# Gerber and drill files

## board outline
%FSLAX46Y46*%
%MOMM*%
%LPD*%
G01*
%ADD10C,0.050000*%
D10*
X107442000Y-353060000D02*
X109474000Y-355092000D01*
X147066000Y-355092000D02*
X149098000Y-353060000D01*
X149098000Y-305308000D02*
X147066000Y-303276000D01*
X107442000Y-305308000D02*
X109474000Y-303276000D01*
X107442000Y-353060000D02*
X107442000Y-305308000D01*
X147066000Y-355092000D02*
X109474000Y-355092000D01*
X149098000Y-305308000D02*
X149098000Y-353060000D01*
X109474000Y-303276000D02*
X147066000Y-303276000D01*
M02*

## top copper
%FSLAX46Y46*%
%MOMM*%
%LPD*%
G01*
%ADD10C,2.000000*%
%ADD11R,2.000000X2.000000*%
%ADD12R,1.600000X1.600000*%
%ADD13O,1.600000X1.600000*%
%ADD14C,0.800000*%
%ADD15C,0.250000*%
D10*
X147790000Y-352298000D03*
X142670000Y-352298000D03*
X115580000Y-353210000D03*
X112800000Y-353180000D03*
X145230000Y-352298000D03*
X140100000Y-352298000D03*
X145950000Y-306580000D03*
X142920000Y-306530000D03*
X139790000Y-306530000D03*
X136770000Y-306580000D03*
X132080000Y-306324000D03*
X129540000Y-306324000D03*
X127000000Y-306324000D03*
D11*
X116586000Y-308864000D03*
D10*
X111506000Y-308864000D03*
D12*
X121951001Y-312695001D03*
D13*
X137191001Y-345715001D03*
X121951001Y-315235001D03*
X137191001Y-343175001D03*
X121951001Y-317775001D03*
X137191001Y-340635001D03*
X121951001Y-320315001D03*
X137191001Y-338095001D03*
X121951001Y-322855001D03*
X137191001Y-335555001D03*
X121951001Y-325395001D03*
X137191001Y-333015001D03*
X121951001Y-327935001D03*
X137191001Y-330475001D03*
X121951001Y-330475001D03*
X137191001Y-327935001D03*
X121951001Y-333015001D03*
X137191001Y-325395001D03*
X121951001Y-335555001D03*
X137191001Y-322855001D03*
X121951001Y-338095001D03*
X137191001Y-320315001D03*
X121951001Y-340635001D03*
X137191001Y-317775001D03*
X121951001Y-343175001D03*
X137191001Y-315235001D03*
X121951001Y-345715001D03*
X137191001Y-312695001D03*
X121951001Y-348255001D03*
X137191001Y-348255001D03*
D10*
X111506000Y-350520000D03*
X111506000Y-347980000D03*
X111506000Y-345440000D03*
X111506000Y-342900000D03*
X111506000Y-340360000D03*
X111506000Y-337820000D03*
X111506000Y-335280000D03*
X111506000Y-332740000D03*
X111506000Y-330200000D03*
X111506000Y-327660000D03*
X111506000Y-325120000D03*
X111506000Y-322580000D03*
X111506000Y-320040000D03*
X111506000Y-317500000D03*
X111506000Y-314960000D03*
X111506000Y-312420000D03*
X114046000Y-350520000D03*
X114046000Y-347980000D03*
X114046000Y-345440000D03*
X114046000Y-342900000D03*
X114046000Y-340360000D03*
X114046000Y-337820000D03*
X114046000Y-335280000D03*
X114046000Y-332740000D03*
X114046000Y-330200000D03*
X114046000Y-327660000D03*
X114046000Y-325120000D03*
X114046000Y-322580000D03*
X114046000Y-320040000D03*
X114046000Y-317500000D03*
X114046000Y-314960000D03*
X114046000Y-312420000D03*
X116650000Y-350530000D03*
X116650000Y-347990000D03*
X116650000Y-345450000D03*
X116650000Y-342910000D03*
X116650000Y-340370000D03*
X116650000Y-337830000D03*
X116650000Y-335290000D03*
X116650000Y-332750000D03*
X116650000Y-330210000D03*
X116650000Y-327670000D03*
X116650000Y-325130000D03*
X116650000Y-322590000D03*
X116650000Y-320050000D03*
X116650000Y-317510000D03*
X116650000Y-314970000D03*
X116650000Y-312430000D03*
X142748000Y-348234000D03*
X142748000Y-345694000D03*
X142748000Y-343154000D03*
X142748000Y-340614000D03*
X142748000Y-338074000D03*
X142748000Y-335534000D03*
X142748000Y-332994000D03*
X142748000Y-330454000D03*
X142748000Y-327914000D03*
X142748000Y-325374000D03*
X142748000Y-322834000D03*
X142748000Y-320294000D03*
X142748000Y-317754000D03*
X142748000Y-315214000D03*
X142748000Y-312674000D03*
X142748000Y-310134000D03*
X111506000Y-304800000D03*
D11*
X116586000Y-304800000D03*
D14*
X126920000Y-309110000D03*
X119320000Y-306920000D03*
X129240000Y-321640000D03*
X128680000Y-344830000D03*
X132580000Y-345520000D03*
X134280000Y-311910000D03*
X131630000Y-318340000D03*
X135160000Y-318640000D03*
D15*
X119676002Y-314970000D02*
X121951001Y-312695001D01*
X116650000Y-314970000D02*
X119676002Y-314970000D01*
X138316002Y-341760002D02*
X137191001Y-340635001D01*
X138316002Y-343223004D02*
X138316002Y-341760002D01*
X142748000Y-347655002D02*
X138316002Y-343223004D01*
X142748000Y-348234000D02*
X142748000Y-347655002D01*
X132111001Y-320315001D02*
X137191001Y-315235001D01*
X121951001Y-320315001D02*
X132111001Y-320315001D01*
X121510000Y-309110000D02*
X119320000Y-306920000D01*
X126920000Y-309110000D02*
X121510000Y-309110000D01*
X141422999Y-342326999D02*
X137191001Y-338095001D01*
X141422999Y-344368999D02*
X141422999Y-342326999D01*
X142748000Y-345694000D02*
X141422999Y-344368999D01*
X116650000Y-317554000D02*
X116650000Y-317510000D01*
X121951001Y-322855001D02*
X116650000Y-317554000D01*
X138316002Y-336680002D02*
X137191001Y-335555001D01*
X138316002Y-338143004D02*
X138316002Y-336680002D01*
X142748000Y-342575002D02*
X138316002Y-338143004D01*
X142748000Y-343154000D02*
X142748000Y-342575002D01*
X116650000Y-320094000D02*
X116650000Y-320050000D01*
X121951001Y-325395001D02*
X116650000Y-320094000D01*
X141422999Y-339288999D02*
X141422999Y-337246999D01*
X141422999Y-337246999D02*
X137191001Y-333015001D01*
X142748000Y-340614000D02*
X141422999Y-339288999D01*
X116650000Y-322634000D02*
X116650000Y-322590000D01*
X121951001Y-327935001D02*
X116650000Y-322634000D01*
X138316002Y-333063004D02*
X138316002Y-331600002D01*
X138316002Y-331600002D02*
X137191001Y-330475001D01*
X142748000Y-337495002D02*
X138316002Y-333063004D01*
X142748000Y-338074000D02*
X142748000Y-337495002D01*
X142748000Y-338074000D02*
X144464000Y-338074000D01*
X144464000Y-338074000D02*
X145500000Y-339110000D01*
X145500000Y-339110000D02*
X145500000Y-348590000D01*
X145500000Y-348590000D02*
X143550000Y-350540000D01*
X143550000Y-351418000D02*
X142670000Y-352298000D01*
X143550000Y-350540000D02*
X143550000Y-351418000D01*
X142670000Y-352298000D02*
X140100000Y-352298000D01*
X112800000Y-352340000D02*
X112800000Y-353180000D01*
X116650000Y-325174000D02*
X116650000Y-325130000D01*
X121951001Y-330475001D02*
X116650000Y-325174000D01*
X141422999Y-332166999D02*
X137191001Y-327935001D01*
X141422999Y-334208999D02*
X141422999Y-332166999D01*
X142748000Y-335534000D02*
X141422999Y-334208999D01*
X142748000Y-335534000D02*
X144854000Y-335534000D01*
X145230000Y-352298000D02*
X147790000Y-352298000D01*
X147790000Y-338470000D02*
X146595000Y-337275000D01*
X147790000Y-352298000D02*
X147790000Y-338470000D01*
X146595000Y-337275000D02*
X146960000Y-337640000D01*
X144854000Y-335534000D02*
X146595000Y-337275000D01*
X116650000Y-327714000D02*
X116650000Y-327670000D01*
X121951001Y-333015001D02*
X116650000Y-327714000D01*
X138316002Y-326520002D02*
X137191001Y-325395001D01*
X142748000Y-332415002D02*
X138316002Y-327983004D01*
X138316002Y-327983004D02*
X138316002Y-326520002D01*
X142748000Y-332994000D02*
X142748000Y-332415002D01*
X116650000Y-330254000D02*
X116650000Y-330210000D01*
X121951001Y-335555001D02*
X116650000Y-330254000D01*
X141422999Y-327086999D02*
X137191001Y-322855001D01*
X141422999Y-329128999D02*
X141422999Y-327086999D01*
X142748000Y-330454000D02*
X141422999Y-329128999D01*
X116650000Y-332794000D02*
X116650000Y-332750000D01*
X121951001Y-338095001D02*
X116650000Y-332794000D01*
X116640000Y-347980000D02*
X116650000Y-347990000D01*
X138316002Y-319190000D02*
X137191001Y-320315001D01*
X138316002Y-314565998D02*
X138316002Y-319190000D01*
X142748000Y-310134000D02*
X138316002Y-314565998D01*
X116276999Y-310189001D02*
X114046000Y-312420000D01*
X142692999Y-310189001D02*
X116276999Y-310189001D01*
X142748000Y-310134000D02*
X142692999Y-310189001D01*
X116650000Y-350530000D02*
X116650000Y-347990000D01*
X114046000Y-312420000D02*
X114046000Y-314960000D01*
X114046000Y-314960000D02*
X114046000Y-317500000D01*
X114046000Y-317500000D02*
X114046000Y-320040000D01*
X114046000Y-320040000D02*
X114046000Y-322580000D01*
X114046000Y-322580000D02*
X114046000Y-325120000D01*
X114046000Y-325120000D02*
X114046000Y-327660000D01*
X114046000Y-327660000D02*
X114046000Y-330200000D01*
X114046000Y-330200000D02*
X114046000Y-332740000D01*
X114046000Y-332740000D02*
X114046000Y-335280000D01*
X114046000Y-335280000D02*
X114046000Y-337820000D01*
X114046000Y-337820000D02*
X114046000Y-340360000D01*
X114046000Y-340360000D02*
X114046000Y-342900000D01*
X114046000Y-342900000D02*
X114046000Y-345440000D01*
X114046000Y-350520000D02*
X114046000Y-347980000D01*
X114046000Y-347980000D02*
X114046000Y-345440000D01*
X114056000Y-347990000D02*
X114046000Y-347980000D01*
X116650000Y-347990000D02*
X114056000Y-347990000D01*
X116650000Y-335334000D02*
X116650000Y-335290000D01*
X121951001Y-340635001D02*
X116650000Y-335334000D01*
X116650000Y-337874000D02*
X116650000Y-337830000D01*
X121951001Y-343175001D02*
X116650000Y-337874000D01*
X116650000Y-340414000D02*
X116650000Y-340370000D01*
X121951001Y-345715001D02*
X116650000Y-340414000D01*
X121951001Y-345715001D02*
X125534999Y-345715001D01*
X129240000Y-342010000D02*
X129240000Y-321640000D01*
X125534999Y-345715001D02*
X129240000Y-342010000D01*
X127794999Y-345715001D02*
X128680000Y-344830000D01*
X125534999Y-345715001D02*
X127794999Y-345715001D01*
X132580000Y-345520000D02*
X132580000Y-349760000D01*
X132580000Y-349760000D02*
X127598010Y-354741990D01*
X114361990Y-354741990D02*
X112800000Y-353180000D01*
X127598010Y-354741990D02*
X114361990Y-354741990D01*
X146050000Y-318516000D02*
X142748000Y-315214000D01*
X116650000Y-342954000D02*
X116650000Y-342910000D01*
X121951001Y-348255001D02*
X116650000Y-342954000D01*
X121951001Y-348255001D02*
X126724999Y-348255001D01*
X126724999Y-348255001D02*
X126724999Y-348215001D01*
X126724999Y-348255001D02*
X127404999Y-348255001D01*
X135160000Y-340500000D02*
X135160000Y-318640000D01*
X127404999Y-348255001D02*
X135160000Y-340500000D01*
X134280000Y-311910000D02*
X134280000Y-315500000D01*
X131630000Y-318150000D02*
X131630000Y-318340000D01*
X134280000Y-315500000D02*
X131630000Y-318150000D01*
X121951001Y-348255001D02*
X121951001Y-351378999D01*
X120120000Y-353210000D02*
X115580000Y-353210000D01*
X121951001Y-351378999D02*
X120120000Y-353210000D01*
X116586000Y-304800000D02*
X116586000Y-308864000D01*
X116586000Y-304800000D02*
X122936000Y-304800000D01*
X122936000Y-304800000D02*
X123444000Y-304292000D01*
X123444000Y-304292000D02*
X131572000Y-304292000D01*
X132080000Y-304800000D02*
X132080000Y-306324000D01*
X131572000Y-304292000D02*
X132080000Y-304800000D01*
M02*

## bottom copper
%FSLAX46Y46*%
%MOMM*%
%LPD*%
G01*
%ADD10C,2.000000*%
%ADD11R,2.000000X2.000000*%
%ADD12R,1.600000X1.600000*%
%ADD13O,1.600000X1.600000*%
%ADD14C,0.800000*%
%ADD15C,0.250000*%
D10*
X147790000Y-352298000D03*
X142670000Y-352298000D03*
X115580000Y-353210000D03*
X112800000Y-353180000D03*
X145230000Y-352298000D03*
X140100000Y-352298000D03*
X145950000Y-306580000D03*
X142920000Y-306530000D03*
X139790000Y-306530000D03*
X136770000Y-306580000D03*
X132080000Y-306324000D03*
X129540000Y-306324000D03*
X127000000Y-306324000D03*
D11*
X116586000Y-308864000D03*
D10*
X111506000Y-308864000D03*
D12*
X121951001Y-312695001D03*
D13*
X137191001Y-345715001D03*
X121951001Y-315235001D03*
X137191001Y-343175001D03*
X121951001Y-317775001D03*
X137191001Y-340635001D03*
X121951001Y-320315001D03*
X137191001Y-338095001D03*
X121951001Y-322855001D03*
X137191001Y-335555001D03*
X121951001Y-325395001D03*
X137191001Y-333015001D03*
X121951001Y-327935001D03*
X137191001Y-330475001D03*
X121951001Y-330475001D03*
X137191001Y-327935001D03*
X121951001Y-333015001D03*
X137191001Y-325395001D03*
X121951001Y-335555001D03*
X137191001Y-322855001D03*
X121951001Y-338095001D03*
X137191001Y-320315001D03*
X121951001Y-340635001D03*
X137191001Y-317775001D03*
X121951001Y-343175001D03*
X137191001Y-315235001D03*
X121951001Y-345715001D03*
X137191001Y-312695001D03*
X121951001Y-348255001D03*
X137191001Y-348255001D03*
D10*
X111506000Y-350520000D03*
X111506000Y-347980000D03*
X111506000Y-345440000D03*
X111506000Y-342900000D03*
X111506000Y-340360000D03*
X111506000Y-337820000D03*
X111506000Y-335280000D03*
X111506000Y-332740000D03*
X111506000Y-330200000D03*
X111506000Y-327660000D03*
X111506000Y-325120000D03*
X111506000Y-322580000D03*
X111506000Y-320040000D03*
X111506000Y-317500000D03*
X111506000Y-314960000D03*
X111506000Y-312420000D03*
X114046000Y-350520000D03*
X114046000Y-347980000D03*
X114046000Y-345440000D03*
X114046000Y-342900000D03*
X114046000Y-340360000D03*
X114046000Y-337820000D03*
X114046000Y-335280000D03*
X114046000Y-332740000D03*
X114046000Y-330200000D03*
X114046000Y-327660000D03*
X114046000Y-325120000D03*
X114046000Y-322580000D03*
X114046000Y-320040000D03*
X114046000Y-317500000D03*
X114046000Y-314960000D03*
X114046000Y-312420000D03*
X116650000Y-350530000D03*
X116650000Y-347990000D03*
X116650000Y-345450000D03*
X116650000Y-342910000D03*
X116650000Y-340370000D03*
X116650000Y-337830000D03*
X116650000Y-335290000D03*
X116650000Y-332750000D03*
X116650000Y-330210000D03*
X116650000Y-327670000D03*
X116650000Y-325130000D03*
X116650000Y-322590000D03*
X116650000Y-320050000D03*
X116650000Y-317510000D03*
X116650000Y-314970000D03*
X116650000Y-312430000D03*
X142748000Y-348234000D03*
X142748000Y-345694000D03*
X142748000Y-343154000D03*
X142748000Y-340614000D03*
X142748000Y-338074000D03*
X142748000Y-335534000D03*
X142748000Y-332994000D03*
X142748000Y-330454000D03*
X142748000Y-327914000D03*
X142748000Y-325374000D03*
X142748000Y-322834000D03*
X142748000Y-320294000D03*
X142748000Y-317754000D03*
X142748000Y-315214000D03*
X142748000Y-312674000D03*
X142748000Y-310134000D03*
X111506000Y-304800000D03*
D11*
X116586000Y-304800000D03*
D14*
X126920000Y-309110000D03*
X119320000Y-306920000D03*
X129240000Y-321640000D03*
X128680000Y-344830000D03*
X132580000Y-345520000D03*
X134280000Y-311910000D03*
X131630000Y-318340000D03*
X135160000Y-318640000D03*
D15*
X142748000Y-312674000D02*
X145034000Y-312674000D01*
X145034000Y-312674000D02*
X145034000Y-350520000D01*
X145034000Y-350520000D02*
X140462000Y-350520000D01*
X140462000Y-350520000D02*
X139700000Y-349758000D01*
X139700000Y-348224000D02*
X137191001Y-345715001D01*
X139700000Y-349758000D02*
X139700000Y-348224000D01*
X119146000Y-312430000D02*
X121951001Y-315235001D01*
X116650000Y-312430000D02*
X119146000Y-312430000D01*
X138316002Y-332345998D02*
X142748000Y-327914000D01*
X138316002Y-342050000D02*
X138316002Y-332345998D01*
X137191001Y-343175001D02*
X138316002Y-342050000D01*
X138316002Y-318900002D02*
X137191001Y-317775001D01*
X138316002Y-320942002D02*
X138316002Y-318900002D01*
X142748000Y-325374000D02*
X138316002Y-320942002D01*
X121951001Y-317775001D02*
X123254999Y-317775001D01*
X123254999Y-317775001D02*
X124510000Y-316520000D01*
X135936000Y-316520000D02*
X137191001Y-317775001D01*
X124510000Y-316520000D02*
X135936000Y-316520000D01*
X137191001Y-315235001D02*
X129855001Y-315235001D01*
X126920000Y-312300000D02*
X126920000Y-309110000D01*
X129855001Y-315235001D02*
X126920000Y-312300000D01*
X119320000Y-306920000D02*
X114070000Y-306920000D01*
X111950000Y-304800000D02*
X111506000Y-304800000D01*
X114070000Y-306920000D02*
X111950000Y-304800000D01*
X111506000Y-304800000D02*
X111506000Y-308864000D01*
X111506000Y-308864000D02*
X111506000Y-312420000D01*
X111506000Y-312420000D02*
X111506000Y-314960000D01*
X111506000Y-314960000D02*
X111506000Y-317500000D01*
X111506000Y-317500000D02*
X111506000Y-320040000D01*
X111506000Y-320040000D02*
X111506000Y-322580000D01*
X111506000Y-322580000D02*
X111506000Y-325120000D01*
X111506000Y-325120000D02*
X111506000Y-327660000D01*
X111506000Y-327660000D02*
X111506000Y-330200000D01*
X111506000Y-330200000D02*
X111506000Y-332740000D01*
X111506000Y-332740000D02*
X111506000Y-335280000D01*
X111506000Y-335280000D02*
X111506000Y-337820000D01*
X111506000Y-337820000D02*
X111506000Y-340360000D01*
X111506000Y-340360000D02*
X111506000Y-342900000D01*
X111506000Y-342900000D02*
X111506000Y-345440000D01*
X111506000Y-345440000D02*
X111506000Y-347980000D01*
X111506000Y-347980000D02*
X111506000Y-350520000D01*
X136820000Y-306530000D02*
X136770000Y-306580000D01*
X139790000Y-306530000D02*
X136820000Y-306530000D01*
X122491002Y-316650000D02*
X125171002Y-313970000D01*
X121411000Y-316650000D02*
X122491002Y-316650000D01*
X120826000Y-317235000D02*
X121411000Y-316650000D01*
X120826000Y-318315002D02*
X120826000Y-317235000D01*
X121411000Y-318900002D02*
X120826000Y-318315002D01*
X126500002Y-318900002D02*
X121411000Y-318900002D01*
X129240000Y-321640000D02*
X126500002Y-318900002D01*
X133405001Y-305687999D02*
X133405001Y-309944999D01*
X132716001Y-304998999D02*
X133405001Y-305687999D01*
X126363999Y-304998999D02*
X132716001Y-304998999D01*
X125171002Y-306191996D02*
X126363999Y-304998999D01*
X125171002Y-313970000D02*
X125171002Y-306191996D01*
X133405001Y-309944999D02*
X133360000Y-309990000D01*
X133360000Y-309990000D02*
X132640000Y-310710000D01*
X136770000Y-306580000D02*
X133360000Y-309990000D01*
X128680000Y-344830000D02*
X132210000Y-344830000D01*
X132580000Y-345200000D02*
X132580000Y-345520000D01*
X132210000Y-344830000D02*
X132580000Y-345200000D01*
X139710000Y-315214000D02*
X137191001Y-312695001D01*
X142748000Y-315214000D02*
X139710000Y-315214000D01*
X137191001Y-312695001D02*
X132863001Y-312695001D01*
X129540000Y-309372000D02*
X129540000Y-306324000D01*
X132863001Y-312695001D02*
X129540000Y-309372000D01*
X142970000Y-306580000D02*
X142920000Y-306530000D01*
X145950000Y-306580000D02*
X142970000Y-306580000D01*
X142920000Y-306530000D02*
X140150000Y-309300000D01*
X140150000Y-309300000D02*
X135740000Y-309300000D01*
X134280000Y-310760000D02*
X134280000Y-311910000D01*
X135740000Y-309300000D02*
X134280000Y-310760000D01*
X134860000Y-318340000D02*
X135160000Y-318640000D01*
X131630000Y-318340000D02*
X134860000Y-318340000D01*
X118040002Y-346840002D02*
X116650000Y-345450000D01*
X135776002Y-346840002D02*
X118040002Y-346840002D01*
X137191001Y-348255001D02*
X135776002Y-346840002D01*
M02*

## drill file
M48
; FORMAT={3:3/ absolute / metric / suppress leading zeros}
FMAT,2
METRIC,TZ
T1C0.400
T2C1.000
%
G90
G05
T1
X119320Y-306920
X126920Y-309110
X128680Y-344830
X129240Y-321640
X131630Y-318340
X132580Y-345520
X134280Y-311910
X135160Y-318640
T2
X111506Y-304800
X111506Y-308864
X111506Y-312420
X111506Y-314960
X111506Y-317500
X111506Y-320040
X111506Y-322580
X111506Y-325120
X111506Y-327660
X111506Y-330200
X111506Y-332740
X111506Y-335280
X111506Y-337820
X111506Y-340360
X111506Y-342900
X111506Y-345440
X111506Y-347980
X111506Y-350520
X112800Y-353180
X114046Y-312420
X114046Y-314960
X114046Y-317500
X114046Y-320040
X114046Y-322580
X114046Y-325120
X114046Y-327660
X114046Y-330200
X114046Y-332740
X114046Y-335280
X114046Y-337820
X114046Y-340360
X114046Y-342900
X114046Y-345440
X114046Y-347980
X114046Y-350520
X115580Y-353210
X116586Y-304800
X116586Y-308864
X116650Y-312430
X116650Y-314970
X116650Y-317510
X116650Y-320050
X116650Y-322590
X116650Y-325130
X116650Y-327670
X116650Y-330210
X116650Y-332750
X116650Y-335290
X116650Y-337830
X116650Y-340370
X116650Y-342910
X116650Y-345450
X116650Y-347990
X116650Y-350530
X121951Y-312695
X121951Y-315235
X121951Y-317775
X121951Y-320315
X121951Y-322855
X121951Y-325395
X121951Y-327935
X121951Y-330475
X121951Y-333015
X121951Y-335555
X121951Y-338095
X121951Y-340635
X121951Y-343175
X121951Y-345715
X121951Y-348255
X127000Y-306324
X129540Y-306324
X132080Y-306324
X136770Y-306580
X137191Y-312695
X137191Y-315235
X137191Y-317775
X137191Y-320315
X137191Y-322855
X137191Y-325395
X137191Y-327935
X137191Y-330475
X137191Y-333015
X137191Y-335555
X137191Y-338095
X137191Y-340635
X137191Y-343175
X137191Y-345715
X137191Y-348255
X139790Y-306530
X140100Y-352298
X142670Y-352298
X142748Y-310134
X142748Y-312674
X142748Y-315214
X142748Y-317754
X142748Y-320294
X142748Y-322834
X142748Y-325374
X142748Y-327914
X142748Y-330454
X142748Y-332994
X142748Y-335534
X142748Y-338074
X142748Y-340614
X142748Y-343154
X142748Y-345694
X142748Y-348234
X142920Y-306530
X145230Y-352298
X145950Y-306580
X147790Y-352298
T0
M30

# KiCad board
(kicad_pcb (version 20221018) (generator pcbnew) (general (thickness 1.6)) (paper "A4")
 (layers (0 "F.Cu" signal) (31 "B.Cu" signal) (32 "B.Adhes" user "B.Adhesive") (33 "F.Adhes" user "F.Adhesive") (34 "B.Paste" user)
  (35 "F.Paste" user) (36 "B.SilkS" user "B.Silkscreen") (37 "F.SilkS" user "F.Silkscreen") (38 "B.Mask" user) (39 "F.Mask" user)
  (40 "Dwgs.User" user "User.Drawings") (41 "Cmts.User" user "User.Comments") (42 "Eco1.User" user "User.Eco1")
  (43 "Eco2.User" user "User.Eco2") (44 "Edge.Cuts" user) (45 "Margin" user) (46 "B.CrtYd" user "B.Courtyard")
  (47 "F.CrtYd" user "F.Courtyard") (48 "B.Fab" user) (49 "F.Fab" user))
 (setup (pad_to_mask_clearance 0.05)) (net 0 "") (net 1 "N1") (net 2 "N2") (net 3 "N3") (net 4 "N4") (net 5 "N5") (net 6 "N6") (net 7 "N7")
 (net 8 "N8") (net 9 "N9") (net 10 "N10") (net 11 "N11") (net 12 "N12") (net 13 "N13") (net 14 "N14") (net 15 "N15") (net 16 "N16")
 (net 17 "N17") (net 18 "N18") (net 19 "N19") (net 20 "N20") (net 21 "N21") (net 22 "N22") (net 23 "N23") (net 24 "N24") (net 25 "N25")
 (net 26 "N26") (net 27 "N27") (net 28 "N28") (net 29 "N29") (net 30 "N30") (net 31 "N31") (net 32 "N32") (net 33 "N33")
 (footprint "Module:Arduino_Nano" (layer "F.Cu") (at 121.951001 312.695001)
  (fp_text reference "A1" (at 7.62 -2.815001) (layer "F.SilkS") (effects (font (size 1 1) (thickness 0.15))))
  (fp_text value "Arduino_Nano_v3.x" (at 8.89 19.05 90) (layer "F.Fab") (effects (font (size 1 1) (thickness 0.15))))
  (pad "1" thru_hole rect (at 0 0) (size 1.6 1.6) (drill 1) (layers "*.Cu" "*.Mask") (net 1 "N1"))
  (pad "2" thru_hole oval (at 0 2.54) (size 1.6 1.6) (drill 1) (layers "*.Cu" "*.Mask") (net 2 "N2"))
  (pad "3" thru_hole oval (at 0 5.08) (size 1.6 1.6) (drill 1) (layers "*.Cu" "*.Mask") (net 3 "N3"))
  (pad "4" thru_hole oval (at 0 7.62) (size 1.6 1.6) (drill 1) (layers "*.Cu" "*.Mask") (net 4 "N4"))
  (pad "5" thru_hole oval (at 0 10.16) (size 1.6 1.6) (drill 1) (layers "*.Cu" "*.Mask") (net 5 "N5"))
  (pad "6" thru_hole oval (at 0 12.7) (size 1.6 1.6) (drill 1) (layers "*.Cu" "*.Mask") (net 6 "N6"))
  (pad "7" thru_hole oval (at 0 15.24) (size 1.6 1.6) (drill 1) (layers "*.Cu" "*.Mask") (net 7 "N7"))
  (pad "8" thru_hole oval (at 0 17.78) (size 1.6 1.6) (drill 1) (layers "*.Cu" "*.Mask") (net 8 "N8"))
  (pad "9" thru_hole oval (at 0 20.32) (size 1.6 1.6) (drill 1) (layers "*.Cu" "*.Mask") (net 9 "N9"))
  (pad "10" thru_hole oval (at 0 22.86) (size 1.6 1.6) (drill 1) (layers "*.Cu" "*.Mask") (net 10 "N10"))
  (pad "11" thru_hole oval (at 0 25.4) (size 1.6 1.6) (drill 1) (layers "*.Cu" "*.Mask") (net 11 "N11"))
  (pad "12" thru_hole oval (at 0 27.94) (size 1.6 1.6) (drill 1) (layers "*.Cu" "*.Mask") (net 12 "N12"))
  (pad "13" thru_hole oval (at 0 30.48) (size 1.6 1.6) (drill 1) (layers "*.Cu" "*.Mask") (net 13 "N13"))
  (pad "14" thru_hole oval (at 0 33.02) (size 1.6 1.6) (drill 1) (layers "*.Cu" "*.Mask") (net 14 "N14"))
  (pad "15" thru_hole oval (at 0 35.56) (size 1.6 1.6) (drill 1) (layers "*.Cu" "*.Mask") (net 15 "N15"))
  (pad "16" thru_hole oval (at 15.24 35.56) (size 1.6 1.6) (drill 1) (layers "*.Cu" "*.Mask") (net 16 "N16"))
  (pad "17" thru_hole oval (at 15.24 33.02) (size 1.6 1.6) (drill 1) (layers "*.Cu" "*.Mask") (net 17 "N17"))
  (pad "18" thru_hole oval (at 15.24 30.48) (size 1.6 1.6) (drill 1) (layers "*.Cu" "*.Mask") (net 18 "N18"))
  (pad "19" thru_hole oval (at 15.24 27.94) (size 1.6 1.6) (drill 1) (layers "*.Cu" "*.Mask") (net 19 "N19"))
  (pad "20" thru_hole oval (at 15.24 25.4) (size 1.6 1.6) (drill 1) (layers "*.Cu" "*.Mask") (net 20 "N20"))
  (pad "21" thru_hole oval (at 15.24 22.86) (size 1.6 1.6) (drill 1) (layers "*.Cu" "*.Mask") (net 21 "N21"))
  (pad "22" thru_hole oval (at 15.24 20.32) (size 1.6 1.6) (drill 1) (layers "*.Cu" "*.Mask") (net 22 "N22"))
  (pad "23" thru_hole oval (at 15.24 17.78) (size 1.6 1.6) (drill 1) (layers "*.Cu" "*.Mask") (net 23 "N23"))
  (pad "24" thru_hole oval (at 15.24 15.24) (size 1.6 1.6) (drill 1) (layers "*.Cu" "*.Mask") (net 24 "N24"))
  (pad "25" thru_hole oval (at 15.24 12.7) (size 1.6 1.6) (drill 1) (layers "*.Cu" "*.Mask") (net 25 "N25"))
  (pad "26" thru_hole oval (at 15.24 10.16) (size 1.6 1.6) (drill 1) (layers "*.Cu" "*.Mask") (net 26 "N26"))
  (pad "27" thru_hole oval (at 15.24 7.62) (size 1.6 1.6) (drill 1) (layers "*.Cu" "*.Mask") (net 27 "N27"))
  (pad "28" thru_hole oval (at 15.24 5.08) (size 1.6 1.6) (drill 1) (layers "*.Cu" "*.Mask") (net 3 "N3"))
  (pad "29" thru_hole oval (at 15.24 2.54) (size 1.6 1.6) (drill 1) (layers "*.Cu" "*.Mask") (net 4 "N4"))
  (pad "30" thru_hole oval (at 15.24 0) (size 1.6 1.6) (drill 1) (layers "*.Cu" "*.Mask") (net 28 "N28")))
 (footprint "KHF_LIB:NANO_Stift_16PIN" (layer "F.Cu") (at 114.046 312.42 -90)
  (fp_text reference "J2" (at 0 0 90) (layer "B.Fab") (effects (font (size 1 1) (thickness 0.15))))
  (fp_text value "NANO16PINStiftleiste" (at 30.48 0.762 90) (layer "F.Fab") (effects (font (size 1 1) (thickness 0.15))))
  (pad "1" thru_hole circle (at 0 0 270) (size 2 2) (drill 1) (layers "*.Cu" "*.Mask") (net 27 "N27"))
  (pad "2" thru_hole circle (at 2.54 0 270) (size 2 2) (drill 1) (layers "*.Cu" "*.Mask") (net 27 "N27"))
  (pad "3" thru_hole circle (at 5.08 0 270) (size 2 2) (drill 1) (layers "*.Cu" "*.Mask") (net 27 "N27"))
  (pad "4" thru_hole circle (at 7.62 0 270) (size 2 2) (drill 1) (layers "*.Cu" "*.Mask") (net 27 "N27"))
  (pad "5" thru_hole circle (at 10.16 0 270) (size 2 2) (drill 1) (layers "*.Cu" "*.Mask") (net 27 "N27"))
  (pad "6" thru_hole circle (at 12.7 0 270) (size 2 2) (drill 1) (layers "*.Cu" "*.Mask") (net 27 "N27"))
  (pad "7" thru_hole circle (at 15.24 0 270) (size 2 2) (drill 1) (layers "*.Cu" "*.Mask") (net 27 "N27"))
  (pad "8" thru_hole circle (at 17.78 0 270) (size 2 2) (drill 1) (layers "*.Cu" "*.Mask") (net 27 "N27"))
  (pad "9" thru_hole circle (at 20.32 0 270) (size 2 2) (drill 1) (layers "*.Cu" "*.Mask") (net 27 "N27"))
  (pad "10" thru_hole circle (at 22.86 0 270) (size 2 2) (drill 1) (layers "*.Cu" "*.Mask") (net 27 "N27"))
  (pad "11" thru_hole circle (at 25.4 0 270) (size 2 2) (drill 1) (layers "*.Cu" "*.Mask") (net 27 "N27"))
  (pad "12" thru_hole circle (at 27.94 0 270) (size 2 2) (drill 1) (layers "*.Cu" "*.Mask") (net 27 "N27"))
  (pad "13" thru_hole circle (at 30.48 0 270) (size 2 2) (drill 1) (layers "*.Cu" "*.Mask") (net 27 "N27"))
  (pad "14" thru_hole circle (at 33.02 0 270) (size 2 2) (drill 1) (layers "*.Cu" "*.Mask") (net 27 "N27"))
  (pad "15" thru_hole circle (at 35.56 0 270) (size 2 2) (drill 1) (layers "*.Cu" "*.Mask") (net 27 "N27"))
  (pad "16" thru_hole circle (at 38.1 0 270) (size 2 2) (drill 1) (layers "*.Cu" "*.Mask") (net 27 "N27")))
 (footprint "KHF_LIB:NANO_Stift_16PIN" (layer "F.Cu") (at 116.65 312.43 -90)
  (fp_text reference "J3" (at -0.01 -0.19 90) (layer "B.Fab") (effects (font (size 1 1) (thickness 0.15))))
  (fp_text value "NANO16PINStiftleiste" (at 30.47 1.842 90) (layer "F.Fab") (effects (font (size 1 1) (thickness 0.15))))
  (pad "1" thru_hole circle (at 0 0 270) (size 2 2) (drill 1) (layers "*.Cu" "*.Mask") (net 2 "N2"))
  (pad "2" thru_hole circle (at 2.54 0 270) (size 2 2) (drill 1) (layers "*.Cu" "*.Mask") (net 1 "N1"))
  (pad "3" thru_hole circle (at 5.08 0 270) (size 2 2) (drill 1) (layers "*.Cu" "*.Mask") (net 5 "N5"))
  (pad "4" thru_hole circle (at 7.62 0 270) (size 2 2) (drill 1) (layers "*.Cu" "*.Mask") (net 6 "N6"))
  (pad "5" thru_hole circle (at 10.16 0 270) (size 2 2) (drill 1) (layers "*.Cu" "*.Mask") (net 7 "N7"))
  (pad "6" thru_hole circle (at 12.7 0 270) (size 2 2) (drill 1) (layers "*.Cu" "*.Mask") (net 8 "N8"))
  (pad "7" thru_hole circle (at 15.24 0 270) (size 2 2) (drill 1) (layers "*.Cu" "*.Mask") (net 9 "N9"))
  (pad "8" thru_hole circle (at 17.78 0 270) (size 2 2) (drill 1) (layers "*.Cu" "*.Mask") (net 10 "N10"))
  (pad "9" thru_hole circle (at 20.32 0 270) (size 2 2) (drill 1) (layers "*.Cu" "*.Mask") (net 11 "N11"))
  (pad "10" thru_hole circle (at 22.86 0 270) (size 2 2) (drill 1) (layers "*.Cu" "*.Mask") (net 12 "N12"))
  (pad "11" thru_hole circle (at 25.4 0 270) (size 2 2) (drill 1) (layers "*.Cu" "*.Mask") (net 13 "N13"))
  (pad "12" thru_hole circle (at 27.94 0 270) (size 2 2) (drill 1) (layers "*.Cu" "*.Mask") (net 14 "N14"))
  (pad "13" thru_hole circle (at 30.48 0 270) (size 2 2) (drill 1) (layers "*.Cu" "*.Mask") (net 15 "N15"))
  (pad "14" thru_hole circle (at 33.02 0 270) (size 2 2) (drill 1) (layers "*.Cu" "*.Mask") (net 16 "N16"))
  (pad "15" thru_hole circle (at 35.56 0 270) (size 2 2) (drill 1) (layers "*.Cu" "*.Mask") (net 27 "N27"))
  (pad "16" thru_hole circle (at 38.1 0 270) (size 2 2) (drill 1) (layers "*.Cu" "*.Mask") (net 27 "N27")))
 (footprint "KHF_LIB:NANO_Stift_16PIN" (layer "F.Cu") (at 142.748 348.234 90)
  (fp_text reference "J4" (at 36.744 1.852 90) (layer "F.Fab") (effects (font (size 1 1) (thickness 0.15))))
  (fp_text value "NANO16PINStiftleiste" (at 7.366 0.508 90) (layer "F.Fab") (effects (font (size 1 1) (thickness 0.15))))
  (pad "1" thru_hole circle (at 0 0 90) (size 2 2) (drill 1) (layers "*.Cu" "*.Mask") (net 19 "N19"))
  (pad "2" thru_hole circle (at 2.54 0 90) (size 2 2) (drill 1) (layers "*.Cu" "*.Mask") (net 20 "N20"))
  (pad "3" thru_hole circle (at 5.08 0 90) (size 2 2) (drill 1) (layers "*.Cu" "*.Mask") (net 21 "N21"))
  (pad "4" thru_hole circle (at 7.62 0 90) (size 2 2) (drill 1) (layers "*.Cu" "*.Mask") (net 22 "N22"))
  (pad "5" thru_hole circle (at 10.16 0 90) (size 2 2) (drill 1) (layers "*.Cu" "*.Mask") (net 23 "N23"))
  (pad "6" thru_hole circle (at 12.7 0 90) (size 2 2) (drill 1) (layers "*.Cu" "*.Mask") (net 24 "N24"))
  (pad "7" thru_hole circle (at 15.24 0 90) (size 2 2) (drill 1) (layers "*.Cu" "*.Mask") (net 25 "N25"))
  (pad "8" thru_hole circle (at 17.78 0 90) (size 2 2) (drill 1) (layers "*.Cu" "*.Mask") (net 26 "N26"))
  (pad "9" thru_hole circle (at 20.32 0 90) (size 2 2) (drill 1) (layers "*.Cu" "*.Mask") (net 18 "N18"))
  (pad "10" thru_hole circle (at 22.86 0 90) (size 2 2) (drill 1) (layers "*.Cu" "*.Mask") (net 3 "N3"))
  (pad "11" thru_hole circle (at 25.4 0 90) (size 2 2) (drill 1) (layers "*.Cu" "*.Mask") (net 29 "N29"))
  (pad "12" thru_hole circle (at 27.94 0 90) (size 2 2) (drill 1) (layers "*.Cu" "*.Mask") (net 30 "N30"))
  (pad "13" thru_hole circle (at 30.48 0 90) (size 2 2) (drill 1) (layers "*.Cu" "*.Mask") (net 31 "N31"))
  (pad "14" thru_hole circle (at 33.02 0 90) (size 2 2) (drill 1) (layers "*.Cu" "*.Mask") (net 28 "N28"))
  (pad "15" thru_hole circle (at 35.56 0 90) (size 2 2) (drill 1) (layers "*.Cu" "*.Mask") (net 17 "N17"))
  (pad "16" thru_hole circle (at 38.1 0 90) (size 2 2) (drill 1) (layers "*.Cu" "*.Mask") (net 27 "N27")))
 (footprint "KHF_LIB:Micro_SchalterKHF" (layer "F.Cu") (at 132.08 306.324 180)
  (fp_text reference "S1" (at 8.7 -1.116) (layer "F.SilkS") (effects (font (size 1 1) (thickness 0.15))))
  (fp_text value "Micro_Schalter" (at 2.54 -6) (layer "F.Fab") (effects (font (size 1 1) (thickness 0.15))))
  (pad "1" thru_hole circle (at 0 0 180) (size 2 2) (drill 1) (layers "*.Cu" "*.Mask") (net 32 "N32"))
  (pad "2" thru_hole circle (at 2.54 0 180) (size 2 2) (drill 1) (layers "*.Cu" "*.Mask") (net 28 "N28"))
  (pad "3" thru_hole circle (at 5.08 0 180) (size 2 2) (drill 1) (layers "*.Cu" "*.Mask") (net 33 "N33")))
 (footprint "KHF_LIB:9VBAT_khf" (layer "F.Cu") (at 111.506 304.8)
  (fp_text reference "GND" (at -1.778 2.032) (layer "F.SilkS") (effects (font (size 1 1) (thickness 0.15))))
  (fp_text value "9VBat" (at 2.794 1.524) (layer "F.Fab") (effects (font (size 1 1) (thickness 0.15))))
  (pad "1" thru_hole circle (at 0 0) (size 2 2) (drill 1) (layers "*.Cu" "*.Mask") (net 4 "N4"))
  (pad "2" thru_hole rect (at 5.08 0) (size 2 2) (drill 1) (layers "*.Cu" "*.Mask") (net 32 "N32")))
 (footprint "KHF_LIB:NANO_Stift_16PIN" (layer "F.Cu") (at 111.506 350.52 90)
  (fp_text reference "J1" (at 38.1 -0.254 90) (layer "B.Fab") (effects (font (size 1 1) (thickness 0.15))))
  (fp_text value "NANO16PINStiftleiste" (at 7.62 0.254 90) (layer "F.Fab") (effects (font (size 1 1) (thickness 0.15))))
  (pad "1" thru_hole circle (at 0 0 90) (size 2 2) (drill 1) (layers "*.Cu" "*.Mask") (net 4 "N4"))
  (pad "2" thru_hole circle (at 2.54 0 90) (size 2 2) (drill 1) (layers "*.Cu" "*.Mask") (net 4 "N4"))
  (pad "3" thru_hole circle (at 5.08 0 90) (size 2 2) (drill 1) (layers "*.Cu" "*.Mask") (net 4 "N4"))
  (pad "4" thru_hole circle (at 7.62 0 90) (size 2 2) (drill 1) (layers "*.Cu" "*.Mask") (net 4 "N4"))
  (pad "5" thru_hole circle (at 10.16 0 90) (size 2 2) (drill 1) (layers "*.Cu" "*.Mask") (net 4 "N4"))
  (pad "6" thru_hole circle (at 12.7 0 90) (size 2 2) (drill 1) (layers "*.Cu" "*.Mask") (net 4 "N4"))
  (pad "7" thru_hole circle (at 15.24 0 90) (size 2 2) (drill 1) (layers "*.Cu" "*.Mask") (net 4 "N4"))
  (pad "8" thru_hole circle (at 17.78 0 90) (size 2 2) (drill 1) (layers "*.Cu" "*.Mask") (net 4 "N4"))
  (pad "9" thru_hole circle (at 20.32 0 90) (size 2 2) (drill 1) (layers "*.Cu" "*.Mask") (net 4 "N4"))
  (pad "10" thru_hole circle (at 22.86 0 90) (size 2 2) (drill 1) (layers "*.Cu" "*.Mask") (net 4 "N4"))
  (pad "11" thru_hole circle (at 25.4 0 90) (size 2 2) (drill 1) (layers "*.Cu" "*.Mask") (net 4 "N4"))
  (pad "12" thru_hole circle (at 27.94 0 90) (size 2 2) (drill 1) (layers "*.Cu" "*.Mask") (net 4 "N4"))
  (pad "13" thru_hole circle (at 30.48 0 90) (size 2 2) (drill 1) (layers "*.Cu" "*.Mask") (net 4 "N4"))
  (pad "14" thru_hole circle (at 33.02 0 90) (size 2 2) (drill 1) (layers "*.Cu" "*.Mask") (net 4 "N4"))
  (pad "15" thru_hole circle (at 35.56 0 90) (size 2 2) (drill 1) (layers "*.Cu" "*.Mask") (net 4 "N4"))
  (pad "16" thru_hole circle (at 38.1 0 90) (size 2 2) (drill 1) (layers "*.Cu" "*.Mask") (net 4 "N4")))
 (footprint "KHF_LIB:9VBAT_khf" (layer "F.Cu") (at 111.506 308.864)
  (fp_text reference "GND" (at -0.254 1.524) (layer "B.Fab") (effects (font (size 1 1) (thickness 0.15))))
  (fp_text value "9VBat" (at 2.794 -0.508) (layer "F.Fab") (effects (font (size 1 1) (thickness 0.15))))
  (pad "1" thru_hole circle (at 0 0) (size 2 2) (drill 1) (layers "*.Cu" "*.Mask") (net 4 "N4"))
  (pad "2" thru_hole rect (at 5.08 0) (size 2 2) (drill 1) (layers "*.Cu" "*.Mask") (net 32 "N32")))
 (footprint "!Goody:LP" (layer "F.Cu") (at 137.31 305.93)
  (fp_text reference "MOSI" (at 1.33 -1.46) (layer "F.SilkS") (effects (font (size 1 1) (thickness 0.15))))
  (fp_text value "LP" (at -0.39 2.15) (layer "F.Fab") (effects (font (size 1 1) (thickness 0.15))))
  (pad "1" thru_hole circle (at -0.54 0.65) (size 2 2) (drill 1) (layers "*.Cu" "*.Mask") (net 14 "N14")))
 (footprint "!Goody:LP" (layer "F.Cu") (at 145.77 351.648)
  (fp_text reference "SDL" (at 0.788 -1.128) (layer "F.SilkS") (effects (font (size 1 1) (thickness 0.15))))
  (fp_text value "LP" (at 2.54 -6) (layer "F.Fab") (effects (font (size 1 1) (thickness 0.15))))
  (pad "1" thru_hole circle (at -0.54 0.65) (size 2 2) (drill 1) (layers "*.Cu" "*.Mask") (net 24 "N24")))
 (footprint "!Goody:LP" (layer "F.Cu") (at 116.12 352.56)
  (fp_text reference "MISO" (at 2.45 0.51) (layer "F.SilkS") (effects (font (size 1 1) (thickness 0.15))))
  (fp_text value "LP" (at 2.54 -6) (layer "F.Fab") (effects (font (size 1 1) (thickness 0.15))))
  (pad "1" thru_hole circle (at -0.54 0.65) (size 2 2) (drill 1) (layers "*.Cu" "*.Mask") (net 15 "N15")))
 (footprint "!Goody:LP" (layer "F.Cu") (at 148.33 351.648)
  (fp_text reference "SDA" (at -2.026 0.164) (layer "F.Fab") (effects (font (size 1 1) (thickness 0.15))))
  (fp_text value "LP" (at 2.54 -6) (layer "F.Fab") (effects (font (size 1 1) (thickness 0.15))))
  (pad "1" thru_hole circle (at -0.54 0.65) (size 2 2) (drill 1) (layers "*.Cu" "*.Mask") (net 24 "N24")))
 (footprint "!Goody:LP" (layer "F.Cu") (at 140.64 351.648)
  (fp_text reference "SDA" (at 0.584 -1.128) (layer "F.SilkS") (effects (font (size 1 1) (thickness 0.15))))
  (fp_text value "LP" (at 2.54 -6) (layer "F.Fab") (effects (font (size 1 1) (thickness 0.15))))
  (pad "1" thru_hole circle (at -0.54 0.65) (size 2 2) (drill 1) (layers "*.Cu" "*.Mask") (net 23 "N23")))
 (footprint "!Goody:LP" (layer "F.Cu") (at 143.21 351.648)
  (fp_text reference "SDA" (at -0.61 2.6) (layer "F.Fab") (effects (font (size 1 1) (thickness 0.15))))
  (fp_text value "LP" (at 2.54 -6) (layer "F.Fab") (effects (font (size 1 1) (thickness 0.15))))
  (pad "1" thru_hole circle (at -0.54 0.65) (size 2 2) (drill 1) (layers "*.Cu" "*.Mask") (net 23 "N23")))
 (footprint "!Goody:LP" (layer "F.Cu") (at 113.34 352.53)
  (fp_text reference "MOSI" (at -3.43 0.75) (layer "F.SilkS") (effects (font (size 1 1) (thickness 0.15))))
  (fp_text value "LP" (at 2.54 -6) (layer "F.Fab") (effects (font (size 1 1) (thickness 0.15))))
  (pad "1" thru_hole circle (at -0.54 0.65) (size 2 2) (drill 1) (layers "*.Cu" "*.Mask") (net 14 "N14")))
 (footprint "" (layer "F.Cu") (at 112.268 348.488)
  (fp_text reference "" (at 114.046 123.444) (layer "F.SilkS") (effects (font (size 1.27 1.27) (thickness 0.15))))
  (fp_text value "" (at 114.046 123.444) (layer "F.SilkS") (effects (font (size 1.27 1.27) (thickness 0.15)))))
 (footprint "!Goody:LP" (layer "F.Cu") (at 146.49 305.93)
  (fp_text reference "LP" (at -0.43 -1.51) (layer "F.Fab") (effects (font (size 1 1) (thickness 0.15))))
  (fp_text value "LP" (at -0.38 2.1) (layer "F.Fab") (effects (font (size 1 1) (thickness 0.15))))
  (pad "1" thru_hole circle (at -0.54 0.65) (size 2 2) (drill 1) (layers "*.Cu" "*.Mask") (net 15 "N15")))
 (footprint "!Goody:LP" (layer "F.Cu") (at 143.46 305.88)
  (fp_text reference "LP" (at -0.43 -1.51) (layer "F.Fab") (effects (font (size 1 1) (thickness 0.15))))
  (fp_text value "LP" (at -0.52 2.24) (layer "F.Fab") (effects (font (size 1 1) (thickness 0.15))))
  (pad "1" thru_hole circle (at -0.54 0.65) (size 2 2) (drill 1) (layers "*.Cu" "*.Mask") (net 15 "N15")))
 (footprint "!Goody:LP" (layer "F.Cu") (at 140.33 305.88)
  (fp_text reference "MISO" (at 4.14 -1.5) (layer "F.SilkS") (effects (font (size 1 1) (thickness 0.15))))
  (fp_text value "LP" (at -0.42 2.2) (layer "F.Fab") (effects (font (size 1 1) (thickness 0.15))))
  (pad "1" thru_hole circle (at -0.54 0.65) (size 2 2) (drill 1) (layers "*.Cu" "*.Mask") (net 14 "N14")))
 (gr_line (start 107.442 353.06) (end 107.442 305.308) (stroke (width 0.05) (type solid)) (layer "Edge.Cuts"))
 (gr_line (start 147.066 355.092) (end 149.098 353.06) (stroke (width 0.05) (type solid)) (layer "Edge.Cuts"))
 (gr_line (start 147.066 355.092) (end 109.474 355.092) (stroke (width 0.05) (type solid)) (layer "Edge.Cuts"))
 (gr_line (start 107.442 305.308) (end 109.474 303.276) (stroke (width 0.05) (type solid)) (layer "Edge.Cuts"))
 (gr_line (start 107.442 353.06) (end 109.474 355.092) (stroke (width 0.05) (type solid)) (layer "Edge.Cuts"))
 (gr_line (start 149.098 305.308) (end 147.066 303.276) (stroke (width 0.05) (type solid)) (layer "Edge.Cuts"))
 (gr_line (start 149.098 305.308) (end 149.098 353.06) (stroke (width 0.05) (type solid)) (layer "Edge.Cuts"))
 (gr_line (start 109.474 303.276) (end 147.066 303.276) (stroke (width 0.05) (type solid)) (layer "Edge.Cuts"))
 (segment (start 119.676002 314.97) (end 121.951001 312.695001) (width 0.25) (layer "F.Cu") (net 1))
 (segment (start 116.65 314.97) (end 119.676002 314.97) (width 0.25) (layer "F.Cu") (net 1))
 (segment (start 140.462 350.52) (end 139.7 349.758) (width 0.25) (layer "B.Cu") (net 17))
 (segment (start 145.034 312.674) (end 145.034 350.52) (width 0.25) (layer "B.Cu") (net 17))
 (segment (start 139.7 348.224) (end 137.191001 345.715001) (width 0.25) (layer "B.Cu") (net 17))
 (segment (start 145.034 350.52) (end 140.462 350.52) (width 0.25) (layer "B.Cu") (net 17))
 (segment (start 142.748 312.674) (end 145.034 312.674) (width 0.25) (layer "B.Cu") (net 17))
 (segment (start 139.7 349.758) (end 139.7 348.224) (width 0.25) (layer "B.Cu") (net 17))
 (segment (start 119.146 312.43) (end 121.951001 315.235001) (width 0.25) (layer "B.Cu") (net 2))
 (segment (start 116.65 312.43) (end 119.146 312.43) (width 0.25) (layer "B.Cu") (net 2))
 (segment (start 137.191001 343.175001) (end 138.316002 342.05) (width 0.25) (layer "B.Cu") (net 18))
 (segment (start 138.316002 332.345998) (end 142.748 327.914) (width 0.25) (layer "B.Cu") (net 18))
 (segment (start 138.316002 342.05) (end 138.316002 332.345998) (width 0.25) (layer "B.Cu") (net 18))
 (segment (start 138.316002 318.900002) (end 137.191001 317.775001) (width 0.25) (layer "B.Cu") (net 3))
 (segment (start 138.316002 320.942002) (end 138.316002 318.900002) (width 0.25) (layer "B.Cu") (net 3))
 (segment (start 123.254999 317.775001) (end 124.51 316.52) (width 0.25) (layer "B.Cu") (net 3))
 (segment (start 121.951001 317.775001) (end 123.254999 317.775001) (width 0.25) (layer "B.Cu") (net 3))
 (segment (start 142.748 325.374) (end 138.316002 320.942002) (width 0.25) (layer "B.Cu") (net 3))
 (segment (start 135.936 316.52) (end 137.191001 317.775001) (width 0.25) (layer "B.Cu") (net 3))
 (segment (start 124.51 316.52) (end 135.936 316.52) (width 0.25) (layer "B.Cu") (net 3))
 (segment (start 142.748 347.655002) (end 138.316002 343.223004) (width 0.25) (layer "F.Cu") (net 19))
 (segment (start 138.316002 343.223004) (end 138.316002 341.760002) (width 0.25) (layer "F.Cu") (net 19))
 (segment (start 142.748 348.234) (end 142.748 347.655002) (width 0.25) (layer "F.Cu") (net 19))
 (segment (start 138.316002 341.760002) (end 137.191001 340.635001) (width 0.25) (layer "F.Cu") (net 19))
 (segment (start 121.951001 320.315001) (end 132.111001 320.315001) (width 0.25) (layer "F.Cu") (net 4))
 (segment (start 132.111001 320.315001) (end 137.191001 315.235001) (width 0.25) (layer "F.Cu") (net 4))
 (segment (start 121.51 309.11) (end 119.32 306.92) (width 0.25) (layer "F.Cu") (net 4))
 (segment (start 126.92 309.11) (end 121.51 309.11) (width 0.25) (layer "F.Cu") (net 4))
 (via (at 126.92 309.11) (size 0.8) (drill 0.4) (layers "F.Cu" "B.Cu") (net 4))
 (via (at 119.32 306.92) (size 0.8) (drill 0.4) (layers "F.Cu" "B.Cu") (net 4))
 (segment (start 111.506 337.82) (end 111.506 340.36) (width 0.25) (layer "B.Cu") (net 4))
 (segment (start 111.95 304.8) (end 111.506 304.8) (width 0.25) (layer "B.Cu") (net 4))
 (segment (start 111.506 308.864) (end 111.506 312.42) (width 0.25) (layer "B.Cu") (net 4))
 (segment (start 114.07 306.92) (end 111.95 304.8) (width 0.25) (layer "B.Cu") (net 4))
 (segment (start 111.506 320.04) (end 111.506 322.58) (width 0.25) (layer "B.Cu") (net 4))
 (segment (start 111.506 332.74) (end 111.506 335.28) (width 0.25) (layer "B.Cu") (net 4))
 (segment (start 111.506 304.8) (end 111.506 308.864) (width 0.25) (layer "B.Cu") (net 4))
 (segment (start 111.506 325.12) (end 111.506 327.66) (width 0.25) (layer "B.Cu") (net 4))
 (segment (start 111.506 342.9) (end 111.506 345.44) (width 0.25) (layer "B.Cu") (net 4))
 (segment (start 111.506 322.58) (end 111.506 325.12) (width 0.25) (layer "B.Cu") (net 4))
 (segment (start 119.32 306.92) (end 114.07 306.92) (width 0.25) (layer "B.Cu") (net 4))
 (segment (start 129.855001 315.235001) (end 126.92 312.3) (width 0.25) (layer "B.Cu") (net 4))
 (segment (start 111.506 314.96) (end 111.506 317.5) (width 0.25) (layer "B.Cu") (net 4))
 (segment (start 111.506 330.2) (end 111.506 332.74) (width 0.25) (layer "B.Cu") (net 4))
 (segment (start 137.191001 315.235001) (end 129.855001 315.235001) (width 0.25) (layer "B.Cu") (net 4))
 (segment (start 111.506 347.98) (end 111.506 350.52) (width 0.25) (layer "B.Cu") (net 4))
 (segment (start 111.506 317.5) (end 111.506 320.04) (width 0.25) (layer "B.Cu") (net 4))
 (segment (start 111.506 345.44) (end 111.506 347.98) (width 0.25) (layer "B.Cu") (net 4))
 (segment (start 111.506 312.42) (end 111.506 314.96) (width 0.25) (layer "B.Cu") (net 4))
 (segment (start 111.506 340.36) (end 111.506 342.9) (width 0.25) (layer "B.Cu") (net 4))
 (segment (start 111.506 335.28) (end 111.506 337.82) (width 0.25) (layer "B.Cu") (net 4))
 (segment (start 111.506 327.66) (end 111.506 330.2) (width 0.25) (layer "B.Cu") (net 4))
 (segment (start 126.92 312.3) (end 126.92 309.11) (width 0.25) (layer "B.Cu") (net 4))
 (segment (start 141.422999 342.326999) (end 137.191001 338.095001) (width 0.25) (layer "F.Cu") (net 20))
 (segment (start 141.422999 344.368999) (end 141.422999 342.326999) (width 0.25) (layer "F.Cu") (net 20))
 (segment (start 142.748 345.694) (end 141.422999 344.368999) (width 0.25) (layer "F.Cu") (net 20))
 (segment (start 121.951001 322.855001) (end 116.65 317.554) (width 0.25) (layer "F.Cu") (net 5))
 (segment (start 116.65 317.554) (end 116.65 317.51) (width 0.25) (layer "F.Cu") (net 5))
 (segment (start 138.316002 336.680002) (end 137.191001 335.555001) (width 0.25) (layer "F.Cu") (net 21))
 (segment (start 138.316002 338.143004) (end 138.316002 336.680002) (width 0.25) (layer "F.Cu") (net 21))
 (segment (start 142.748 343.154) (end 142.748 342.575002) (width 0.25) (layer "F.Cu") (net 21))
 (segment (start 142.748 342.575002) (end 138.316002 338.143004) (width 0.25) (layer "F.Cu") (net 21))
 (segment (start 116.65 320.094) (end 116.65 320.05) (width 0.25) (layer "F.Cu") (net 6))
 (segment (start 121.951001 325.395001) (end 116.65 320.094) (width 0.25) (layer "F.Cu") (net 6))
 (segment (start 142.748 340.614) (end 141.422999 339.288999) (width 0.25) (layer "F.Cu") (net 22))
 (segment (start 141.422999 337.246999) (end 137.191001 333.015001) (width 0.25) (layer "F.Cu") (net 22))
 (segment (start 141.422999 339.288999) (end 141.422999 337.246999) (width 0.25) (layer "F.Cu") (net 22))
 (segment (start 116.65 322.634) (end 116.65 322.59) (width 0.25) (layer "F.Cu") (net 7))
 (segment (start 121.951001 327.935001) (end 116.65 322.634) (width 0.25) (layer "F.Cu") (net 7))
 (segment (start 142.67 352.298) (end 140.1 352.298) (width 0.25) (layer "F.Cu") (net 23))
 (segment (start 142.748 337.495002) (end 138.316002 333.063004) (width 0.25) (layer "F.Cu") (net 23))
 (segment (start 145.5 339.11) (end 145.5 348.59) (width 0.25) (layer "F.Cu") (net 23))
 (segment (start 143.55 350.54) (end 143.55 351.418) (width 0.25) (layer "F.Cu") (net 23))
 (segment (start 142.748 338.074) (end 144.464 338.074) (width 0.25) (layer "F.Cu") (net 23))
 (segment (start 144.464 338.074) (end 145.5 339.11) (width 0.25) (layer "F.Cu") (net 23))
 (segment (start 142.748 338.074) (end 142.748 337.495002) (width 0.25) (layer "F.Cu") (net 23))
 (segment (start 138.316002 333.063004) (end 138.316002 331.600002) (width 0.25) (layer "F.Cu") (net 23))
 (segment (start 138.316002 331.600002) (end 137.191001 330.475001) (width 0.25) (layer "F.Cu") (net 23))
 (segment (start 143.55 351.418) (end 142.67 352.298) (width 0.25) (layer "F.Cu") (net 23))
 (segment (start 145.5 348.59) (end 143.55 350.54) (width 0.25) (layer "F.Cu") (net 23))
 (segment (start 116.65 325.174) (end 116.65 325.13) (width 0.25) (layer "F.Cu") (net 8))
 (segment (start 121.951001 330.475001) (end 116.65 325.174) (width 0.25) (layer "F.Cu") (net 8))
 (segment (start 141.422999 332.166999) (end 137.191001 327.935001) (width 0.25) (layer "F.Cu") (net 24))
 (segment (start 146.595 337.275) (end 146.96 337.64) (width 0.25) (layer "F.Cu") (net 24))
 (segment (start 145.23 352.298) (end 147.79 352.298) (width 0.25) (layer "F.Cu") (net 24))
 (segment (start 142.748 335.534) (end 141.422999 334.208999) (width 0.25) (layer "F.Cu") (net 24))
 (segment (start 147.79 338.47) (end 146.595 337.275) (width 0.25) (layer "F.Cu") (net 24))
 (segment (start 147.79 352.298) (end 147.79 338.47) (width 0.25) (layer "F.Cu") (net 24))
 (segment (start 141.422999 334.208999) (end 141.422999 332.166999) (width 0.25) (layer "F.Cu") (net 24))
 (segment (start 142.748 335.534) (end 144.854 335.534) (width 0.25) (layer "F.Cu") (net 24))
 (segment (start 144.854 335.534) (end 146.595 337.275) (width 0.25) (layer "F.Cu") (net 24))
 (segment (start 121.951001 333.015001) (end 116.65 327.714) (width 0.25) (layer "F.Cu") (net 9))
 (segment (start 116.65 327.714) (end 116.65 327.67) (width 0.25) (layer "F.Cu") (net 9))
 (segment (start 142.748 332.994) (end 142.748 332.415002) (width 0.25) (layer "F.Cu") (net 25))
 (segment (start 138.316002 326.520002) (end 137.191001 325.395001) (width 0.25) (layer "F.Cu") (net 25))
 (segment (start 138.316002 327.983004) (end 138.316002 326.520002) (width 0.25) (layer "F.Cu") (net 25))
 (segment (start 142.748 332.415002) (end 138.316002 327.983004) (width 0.25) (layer "F.Cu") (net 25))
 (segment (start 121.951001 335.555001) (end 116.65 330.254) (width 0.25) (layer "F.Cu") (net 10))
 (segment (start 116.65 330.254) (end 116.65 330.21) (width 0.25) (layer "F.Cu") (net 10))
 (segment (start 141.422999 327.086999) (end 137.191001 322.855001) (width 0.25) (layer "F.Cu") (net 26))
 (segment (start 141.422999 329.128999) (end 141.422999 327.086999) (width 0.25) (layer "F.Cu") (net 26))
 (segment (start 142.748 330.454) (end 141.422999 329.128999) (width 0.25) (layer "F.Cu") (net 26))
 (segment (start 116.65 332.794) (end 116.65 332.75) (width 0.25) (layer "F.Cu") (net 11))
 (segment (start 121.951001 338.095001) (end 116.65 332.794) (width 0.25) (layer "F.Cu") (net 11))
 (segment (start 116.276999 310.189001) (end 114.046 312.42) (width 0.25) (layer "F.Cu") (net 27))
 (segment (start 114.046 317.5) (end 114.046 320.04) (width 0.25) (layer "F.Cu") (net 27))
 (segment (start 142.748 310.134) (end 142.692999 310.189001) (width 0.25) (layer "F.Cu") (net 27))
 (segment (start 114.046 342.9) (end 114.046 345.44) (width 0.25) (layer "F.Cu") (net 27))
 (segment (start 114.046 322.58) (end 114.046 325.12) (width 0.25) (layer "F.Cu") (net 27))
 (segment (start 138.316002 314.565998) (end 138.316002 319.19) (width 0.25) (layer "F.Cu") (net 27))
 (segment (start 114.046 327.66) (end 114.046 330.2) (width 0.25) (layer "F.Cu") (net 27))
 (segment (start 114.046 335.28) (end 114.046 337.82) (width 0.25) (layer "F.Cu") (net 27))
 (segment (start 114.046 314.96) (end 114.046 317.5) (width 0.25) (layer "F.Cu") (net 27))
 (segment (start 114.046 347.98) (end 114.046 345.44) (width 0.25) (layer "F.Cu") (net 27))
 (segment (start 114.046 330.2) (end 114.046 332.74) (width 0.25) (layer "F.Cu") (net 27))
 (segment (start 114.046 320.04) (end 114.046 322.58) (width 0.25) (layer "F.Cu") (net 27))
 (segment (start 116.65 350.53) (end 116.65 347.99) (width 0.25) (layer "F.Cu") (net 27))
 (segment (start 114.046 332.74) (end 114.046 335.28) (width 0.25) (layer "F.Cu") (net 27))
 (segment (start 116.64 347.98) (end 116.65 347.99) (width 0.25) (layer "F.Cu") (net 27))
 (segment (start 114.046 337.82) (end 114.046 340.36) (width 0.25) (layer "F.Cu") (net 27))
 (segment (start 142.692999 310.189001) (end 116.276999 310.189001) (width 0.25) (layer "F.Cu") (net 27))
 (segment (start 138.316002 319.19) (end 137.191001 320.315001) (width 0.25) (layer "F.Cu") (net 27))
 (segment (start 142.748 310.134) (end 138.316002 314.565998) (width 0.25) (layer "F.Cu") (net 27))
 (segment (start 114.046 325.12) (end 114.046 327.66) (width 0.25) (layer "F.Cu") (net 27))
 (segment (start 114.056 347.99) (end 114.046 347.98) (width 0.25) (layer "F.Cu") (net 27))
 (segment (start 114.046 340.36) (end 114.046 342.9) (width 0.25) (layer "F.Cu") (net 27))
 (segment (start 116.65 347.99) (end 114.056 347.99) (width 0.25) (layer "F.Cu") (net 27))
 (segment (start 114.046 312.42) (end 114.046 314.96) (width 0.25) (layer "F.Cu") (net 27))
 (segment (start 114.046 350.52) (end 114.046 347.98) (width 0.25) (layer "F.Cu") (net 27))
 (segment (start 116.65 335.334) (end 116.65 335.29) (width 0.25) (layer "F.Cu") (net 12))
 (segment (start 121.951001 340.635001) (end 116.65 335.334) (width 0.25) (layer "F.Cu") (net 12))
 (segment (start 116.65 337.874) (end 116.65 337.83) (width 0.25) (layer "F.Cu") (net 13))
 (segment (start 121.951001 343.175001) (end 116.65 337.874) (width 0.25) (layer "F.Cu") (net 13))
 (segment (start 132.58 345.52) (end 132.58 349.76) (width 0.25) (layer "F.Cu") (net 14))
 (segment (start 116.65 340.414) (end 116.65 340.37) (width 0.25) (layer "F.Cu") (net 14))
 (segment (start 127.59801 354.74199) (end 114.36199 354.74199) (width 0.25) (layer "F.Cu") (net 14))
 (segment (start 125.534999 345.715001) (end 127.794999 345.715001) (width 0.25) (layer "F.Cu") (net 14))
 (segment (start 129.24 342.01) (end 129.24 321.64) (width 0.25) (layer "F.Cu") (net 14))
 (segment (start 127.794999 345.715001) (end 128.68 344.83) (width 0.25) (layer "F.Cu") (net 14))
 (segment (start 114.36199 354.74199) (end 112.8 353.18) (width 0.25) (layer "F.Cu") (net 14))
 (segment (start 121.951001 345.715001) (end 116.65 340.414) (width 0.25) (layer "F.Cu") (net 14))
 (segment (start 125.534999 345.715001) (end 129.24 342.01) (width 0.25) (layer "F.Cu") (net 14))
 (segment (start 121.951001 345.715001) (end 125.534999 345.715001) (width 0.25) (layer "F.Cu") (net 14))
 (segment (start 132.58 349.76) (end 127.59801 354.74199) (width 0.25) (layer "F.Cu") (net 14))
 (segment (start 112.8 352.34) (end 112.8 353.18) (width 0.25) (layer "F.Cu") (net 14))
 (via (at 129.24 321.64) (size 0.8) (drill 0.4) (layers "F.Cu" "B.Cu") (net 14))
 (via (at 128.68 344.83) (size 0.8) (drill 0.4) (layers "F.Cu" "B.Cu") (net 14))
 (via (at 132.58 345.52) (size 0.8) (drill 0.4) (layers "F.Cu" "B.Cu") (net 14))
 (segment (start 132.21 344.83) (end 132.58 345.2) (width 0.25) (layer "B.Cu") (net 14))
 (segment (start 120.826 318.315002) (end 120.826 317.235) (width 0.25) (layer "B.Cu") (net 14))
 (segment (start 132.716001 304.998999) (end 133.405001 305.687999) (width 0.25) (layer "B.Cu") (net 14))
 (segment (start 121.411 318.900002) (end 120.826 318.315002) (width 0.25) (layer "B.Cu") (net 14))
 (segment (start 133.405001 305.687999) (end 133.405001 309.944999) (width 0.25) (layer "B.Cu") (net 14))
 (segment (start 125.171002 306.191996) (end 126.363999 304.998999) (width 0.25) (layer "B.Cu") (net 14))
 (segment (start 128.68 344.83) (end 132.21 344.83) (width 0.25) (layer "B.Cu") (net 14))
 (segment (start 136.77 306.58) (end 133.36 309.99) (width 0.25) (layer "B.Cu") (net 14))
 (segment (start 120.826 317.235) (end 121.411 316.65) (width 0.25) (layer "B.Cu") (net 14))
 (segment (start 129.24 321.64) (end 126.500002 318.900002) (width 0.25) (layer "B.Cu") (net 14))
 (segment (start 125.171002 313.97) (end 125.171002 306.191996) (width 0.25) (layer "B.Cu") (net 14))
 (segment (start 126.363999 304.998999) (end 132.716001 304.998999) (width 0.25) (layer "B.Cu") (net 14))
 (segment (start 121.411 316.65) (end 122.491002 316.65) (width 0.25) (layer "B.Cu") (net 14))
 (segment (start 133.36 309.99) (end 132.64 310.71) (width 0.25) (layer "B.Cu") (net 14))
 (segment (start 132.58 345.2) (end 132.58 345.52) (width 0.25) (layer "B.Cu") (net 14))
 (segment (start 136.82 306.53) (end 136.77 306.58) (width 0.25) (layer "B.Cu") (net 14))
 (segment (start 133.405001 309.944999) (end 133.36 309.99) (width 0.25) (layer "B.Cu") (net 14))
 (segment (start 139.79 306.53) (end 136.82 306.53) (width 0.25) (layer "B.Cu") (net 14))
 (segment (start 122.491002 316.65) (end 125.171002 313.97) (width 0.25) (layer "B.Cu") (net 14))
 (segment (start 126.500002 318.900002) (end 121.411 318.900002) (width 0.25) (layer "B.Cu") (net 14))
 (segment (start 146.05 318.516) (end 142.748 315.214) (width 0.25) (layer "F.Cu") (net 28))
 (segment (start 137.191001 312.695001) (end 132.863001 312.695001) (width 0.25) (layer "B.Cu") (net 28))
 (segment (start 139.71 315.214) (end 137.191001 312.695001) (width 0.25) (layer "B.Cu") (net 28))
 (segment (start 132.863001 312.695001) (end 129.54 309.372) (width 0.25) (layer "B.Cu") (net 28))
 (segment (start 142.748 315.214) (end 139.71 315.214) (width 0.25) (layer "B.Cu") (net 28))
 (segment (start 129.54 309.372) (end 129.54 306.324) (width 0.25) (layer "B.Cu") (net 28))
 (segment (start 134.28 315.5) (end 131.63 318.15) (width 0.25) (layer "F.Cu") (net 15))
 (segment (start 131.63 318.15) (end 131.63 318.34) (width 0.25) (layer "F.Cu") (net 15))
 (segment (start 127.404999 348.255001) (end 135.16 340.5) (width 0.25) (layer "F.Cu") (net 15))
 (segment (start 121.951001 348.255001) (end 121.951001 351.378999) (width 0.25) (layer "F.Cu") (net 15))
 (segment (start 120.12 353.21) (end 115.58 353.21) (width 0.25) (layer "F.Cu") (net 15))
 (segment (start 126.724999 348.255001) (end 126.724999 348.215001) (width 0.25) (layer "F.Cu") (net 15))
 (segment (start 116.65 342.954) (end 116.65 342.91) (width 0.25) (layer "F.Cu") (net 15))
 (segment (start 121.951001 348.255001) (end 126.724999 348.255001) (width 0.25) (layer "F.Cu") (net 15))
 (segment (start 135.16 340.5) (end 135.16 318.64) (width 0.25) (layer "F.Cu") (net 15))
 (segment (start 126.724999 348.255001) (end 127.404999 348.255001) (width 0.25) (layer "F.Cu") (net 15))
 (segment (start 121.951001 351.378999) (end 120.12 353.21) (width 0.25) (layer "F.Cu") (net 15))
 (segment (start 121.951001 348.255001) (end 116.65 342.954) (width 0.25) (layer "F.Cu") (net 15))
 (segment (start 134.28 311.91) (end 134.28 315.5) (width 0.25) (layer "F.Cu") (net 15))
 (via (at 131.63 318.34) (size 0.8) (drill 0.4) (layers "F.Cu" "B.Cu") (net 15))
 (via (at 135.16 318.64) (size 0.8) (drill 0.4) (layers "F.Cu" "B.Cu") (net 15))
 (via (at 134.28 311.91) (size 0.8) (drill 0.4) (layers "F.Cu" "B.Cu") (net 15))
 (segment (start 145.95 306.58) (end 142.97 306.58) (width 0.25) (layer "B.Cu") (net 15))
 (segment (start 142.92 306.53) (end 140.15 309.3) (width 0.25) (layer "B.Cu") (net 15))
 (segment (start 131.63 318.34) (end 134.86 318.34) (width 0.25) (layer "B.Cu") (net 15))
 (segment (start 134.86 318.34) (end 135.16 318.64) (width 0.25) (layer "B.Cu") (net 15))
 (segment (start 134.28 310.76) (end 134.28 311.91) (width 0.25) (layer "B.Cu") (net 15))
 (segment (start 140.15 309.3) (end 135.74 309.3) (width 0.25) (layer "B.Cu") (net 15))
 (segment (start 142.97 306.58) (end 142.92 306.53) (width 0.25) (layer "B.Cu") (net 15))
 (segment (start 135.74 309.3) (end 134.28 310.76) (width 0.25) (layer "B.Cu") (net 15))
 (segment (start 137.191001 348.255001) (end 135.776002 346.840002) (width 0.25) (layer "B.Cu") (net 16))
 (segment (start 135.776002 346.840002) (end 118.040002 346.840002) (width 0.25) (layer "B.Cu") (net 16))
 (segment (start 118.040002 346.840002) (end 116.65 345.45) (width 0.25) (layer "B.Cu") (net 16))
 (segment (start 132.08 304.8) (end 132.08 306.324) (width 0.25) (layer "F.Cu") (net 32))
 (segment (start 116.586 304.8) (end 116.586 308.864) (width 0.25) (layer "F.Cu") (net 32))
 (segment (start 131.572 304.292) (end 132.08 304.8) (width 0.25) (layer "F.Cu") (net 32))
 (segment (start 122.936 304.8) (end 123.444 304.292) (width 0.25) (layer "F.Cu") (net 32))
 (segment (start 116.586 304.8) (end 122.936 304.8) (width 0.25) (layer "F.Cu") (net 32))
 (segment (start 123.444 304.292) (end 131.572 304.292) (width 0.25) (layer "F.Cu") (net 32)))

